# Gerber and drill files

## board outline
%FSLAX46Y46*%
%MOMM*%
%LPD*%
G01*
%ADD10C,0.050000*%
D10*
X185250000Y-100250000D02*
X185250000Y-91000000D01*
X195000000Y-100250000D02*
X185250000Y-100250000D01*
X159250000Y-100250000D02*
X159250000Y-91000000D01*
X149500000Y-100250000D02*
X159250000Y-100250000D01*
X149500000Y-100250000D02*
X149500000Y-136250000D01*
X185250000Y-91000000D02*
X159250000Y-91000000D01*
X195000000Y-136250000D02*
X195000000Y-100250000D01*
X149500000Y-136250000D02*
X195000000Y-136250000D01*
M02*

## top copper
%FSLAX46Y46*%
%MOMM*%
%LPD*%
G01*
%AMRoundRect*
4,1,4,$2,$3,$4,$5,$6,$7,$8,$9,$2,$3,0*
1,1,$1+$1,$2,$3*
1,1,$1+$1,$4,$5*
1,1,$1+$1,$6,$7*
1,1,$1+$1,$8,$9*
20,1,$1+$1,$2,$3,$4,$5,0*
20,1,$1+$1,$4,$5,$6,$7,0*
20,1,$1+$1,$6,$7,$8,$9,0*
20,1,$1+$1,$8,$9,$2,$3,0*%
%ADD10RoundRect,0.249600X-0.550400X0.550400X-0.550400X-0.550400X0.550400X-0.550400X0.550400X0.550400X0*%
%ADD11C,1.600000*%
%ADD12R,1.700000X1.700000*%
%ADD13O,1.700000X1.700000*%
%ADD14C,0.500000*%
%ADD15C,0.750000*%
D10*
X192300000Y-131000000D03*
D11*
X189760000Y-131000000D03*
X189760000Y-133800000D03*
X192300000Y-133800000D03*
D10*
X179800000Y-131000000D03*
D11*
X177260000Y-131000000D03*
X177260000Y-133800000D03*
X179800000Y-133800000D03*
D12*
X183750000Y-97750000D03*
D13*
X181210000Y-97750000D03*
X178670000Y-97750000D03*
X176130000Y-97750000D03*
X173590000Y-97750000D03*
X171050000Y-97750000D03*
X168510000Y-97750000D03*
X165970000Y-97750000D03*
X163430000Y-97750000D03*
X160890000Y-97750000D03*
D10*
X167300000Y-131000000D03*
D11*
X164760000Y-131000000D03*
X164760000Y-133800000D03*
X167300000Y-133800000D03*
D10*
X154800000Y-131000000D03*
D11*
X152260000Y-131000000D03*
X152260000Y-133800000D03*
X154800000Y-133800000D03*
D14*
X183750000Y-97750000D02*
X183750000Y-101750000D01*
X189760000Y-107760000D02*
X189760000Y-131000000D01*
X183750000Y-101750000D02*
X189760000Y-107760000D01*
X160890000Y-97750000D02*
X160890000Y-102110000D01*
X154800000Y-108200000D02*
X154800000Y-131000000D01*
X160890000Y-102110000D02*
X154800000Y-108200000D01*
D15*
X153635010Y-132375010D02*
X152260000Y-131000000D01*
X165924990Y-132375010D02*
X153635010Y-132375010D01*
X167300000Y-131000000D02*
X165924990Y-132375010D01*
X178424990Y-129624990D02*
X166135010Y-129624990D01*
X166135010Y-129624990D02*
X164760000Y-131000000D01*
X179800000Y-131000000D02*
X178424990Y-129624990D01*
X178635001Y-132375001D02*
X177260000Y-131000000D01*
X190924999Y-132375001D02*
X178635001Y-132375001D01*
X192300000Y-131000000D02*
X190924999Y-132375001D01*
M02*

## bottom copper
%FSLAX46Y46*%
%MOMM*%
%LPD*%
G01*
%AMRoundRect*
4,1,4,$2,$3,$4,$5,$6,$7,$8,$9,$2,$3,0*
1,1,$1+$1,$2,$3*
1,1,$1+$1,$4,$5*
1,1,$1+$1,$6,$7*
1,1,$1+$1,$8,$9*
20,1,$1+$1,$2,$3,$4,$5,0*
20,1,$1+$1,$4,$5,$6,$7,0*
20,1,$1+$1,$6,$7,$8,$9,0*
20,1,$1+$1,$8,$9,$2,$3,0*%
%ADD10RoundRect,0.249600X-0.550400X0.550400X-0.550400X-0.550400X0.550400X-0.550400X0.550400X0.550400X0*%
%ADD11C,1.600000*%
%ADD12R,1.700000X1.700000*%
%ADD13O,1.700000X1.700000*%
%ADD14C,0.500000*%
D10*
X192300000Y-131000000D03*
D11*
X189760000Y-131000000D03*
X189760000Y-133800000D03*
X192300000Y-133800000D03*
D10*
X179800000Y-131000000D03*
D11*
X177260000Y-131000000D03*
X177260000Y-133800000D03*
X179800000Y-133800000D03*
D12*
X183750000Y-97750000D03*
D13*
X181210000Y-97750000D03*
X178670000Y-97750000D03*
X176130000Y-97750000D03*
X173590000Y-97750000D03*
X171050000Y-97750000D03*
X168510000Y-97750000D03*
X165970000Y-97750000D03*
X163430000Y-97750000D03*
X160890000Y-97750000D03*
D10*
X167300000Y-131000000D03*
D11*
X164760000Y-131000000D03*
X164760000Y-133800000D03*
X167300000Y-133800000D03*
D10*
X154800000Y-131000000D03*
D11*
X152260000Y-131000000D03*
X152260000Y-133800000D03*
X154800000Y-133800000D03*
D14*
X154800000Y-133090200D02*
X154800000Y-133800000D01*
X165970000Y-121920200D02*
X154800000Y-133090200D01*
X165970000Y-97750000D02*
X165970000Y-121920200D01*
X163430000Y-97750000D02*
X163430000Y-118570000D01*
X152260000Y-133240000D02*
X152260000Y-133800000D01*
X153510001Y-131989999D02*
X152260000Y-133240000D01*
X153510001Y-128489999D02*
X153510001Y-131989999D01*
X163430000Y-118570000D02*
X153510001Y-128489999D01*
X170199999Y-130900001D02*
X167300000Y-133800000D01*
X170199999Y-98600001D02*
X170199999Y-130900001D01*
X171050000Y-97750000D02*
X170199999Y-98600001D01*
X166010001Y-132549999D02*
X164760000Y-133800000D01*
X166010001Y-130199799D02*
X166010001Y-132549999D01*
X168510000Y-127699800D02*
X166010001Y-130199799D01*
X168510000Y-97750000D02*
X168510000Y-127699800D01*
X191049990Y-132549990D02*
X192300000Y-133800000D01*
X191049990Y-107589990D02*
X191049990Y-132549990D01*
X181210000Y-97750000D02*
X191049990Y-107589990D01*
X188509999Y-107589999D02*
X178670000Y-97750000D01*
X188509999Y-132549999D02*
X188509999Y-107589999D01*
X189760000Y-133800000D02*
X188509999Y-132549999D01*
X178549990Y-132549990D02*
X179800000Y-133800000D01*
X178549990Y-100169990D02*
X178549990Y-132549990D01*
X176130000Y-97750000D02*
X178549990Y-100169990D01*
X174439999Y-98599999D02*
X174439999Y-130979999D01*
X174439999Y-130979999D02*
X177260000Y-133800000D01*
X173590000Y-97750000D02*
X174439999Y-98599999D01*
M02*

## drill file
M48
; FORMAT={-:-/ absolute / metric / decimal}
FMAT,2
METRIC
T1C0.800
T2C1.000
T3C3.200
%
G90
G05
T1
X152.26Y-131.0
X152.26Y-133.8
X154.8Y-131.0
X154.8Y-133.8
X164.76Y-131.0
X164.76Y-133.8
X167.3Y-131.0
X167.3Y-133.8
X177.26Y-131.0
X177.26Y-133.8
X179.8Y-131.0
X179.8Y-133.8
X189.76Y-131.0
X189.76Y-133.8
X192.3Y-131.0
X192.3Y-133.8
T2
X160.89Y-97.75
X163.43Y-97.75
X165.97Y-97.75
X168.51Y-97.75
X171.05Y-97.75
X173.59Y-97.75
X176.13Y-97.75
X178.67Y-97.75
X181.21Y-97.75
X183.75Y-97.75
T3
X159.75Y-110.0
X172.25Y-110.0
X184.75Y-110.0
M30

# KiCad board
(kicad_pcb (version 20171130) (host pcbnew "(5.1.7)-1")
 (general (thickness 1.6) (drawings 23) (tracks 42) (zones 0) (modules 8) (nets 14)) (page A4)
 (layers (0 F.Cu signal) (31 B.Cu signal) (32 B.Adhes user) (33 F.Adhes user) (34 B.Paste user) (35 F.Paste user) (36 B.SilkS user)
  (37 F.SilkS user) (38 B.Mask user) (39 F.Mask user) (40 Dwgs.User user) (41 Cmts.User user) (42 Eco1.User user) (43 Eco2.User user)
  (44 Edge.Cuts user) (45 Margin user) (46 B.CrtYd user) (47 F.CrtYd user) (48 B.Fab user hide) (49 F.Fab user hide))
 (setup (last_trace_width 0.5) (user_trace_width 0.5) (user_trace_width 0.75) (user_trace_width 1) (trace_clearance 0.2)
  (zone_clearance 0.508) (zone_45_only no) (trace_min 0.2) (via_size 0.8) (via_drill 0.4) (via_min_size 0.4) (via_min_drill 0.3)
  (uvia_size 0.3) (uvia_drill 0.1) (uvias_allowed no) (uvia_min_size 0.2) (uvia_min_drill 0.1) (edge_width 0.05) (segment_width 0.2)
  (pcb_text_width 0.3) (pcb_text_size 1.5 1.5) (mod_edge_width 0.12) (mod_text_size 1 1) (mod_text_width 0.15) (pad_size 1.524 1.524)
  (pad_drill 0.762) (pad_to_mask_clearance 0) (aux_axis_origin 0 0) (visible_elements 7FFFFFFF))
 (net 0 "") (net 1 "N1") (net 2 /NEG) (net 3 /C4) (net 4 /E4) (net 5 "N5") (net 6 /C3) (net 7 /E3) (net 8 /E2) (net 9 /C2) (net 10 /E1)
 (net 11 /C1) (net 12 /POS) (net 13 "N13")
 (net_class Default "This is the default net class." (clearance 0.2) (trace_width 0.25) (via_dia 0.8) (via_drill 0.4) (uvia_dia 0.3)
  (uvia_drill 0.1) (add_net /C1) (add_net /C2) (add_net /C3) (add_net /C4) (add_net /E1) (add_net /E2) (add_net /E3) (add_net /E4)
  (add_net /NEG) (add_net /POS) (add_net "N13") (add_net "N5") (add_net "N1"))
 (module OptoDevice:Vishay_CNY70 (layer F.Cu) (at 192.3 131 270)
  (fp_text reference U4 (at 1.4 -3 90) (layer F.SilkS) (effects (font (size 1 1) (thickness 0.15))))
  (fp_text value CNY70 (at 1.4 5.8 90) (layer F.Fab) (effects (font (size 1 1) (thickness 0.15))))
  (pad 1 thru_hole roundrect (at 0 0 270) (size 1.6 1.6) (drill 0.8) (layers *.Cu *.Mask) (roundrect_rratio 0.156) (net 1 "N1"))
  (pad 2 thru_hole circle (at 0 2.54 270) (size 1.6 1.6) (drill 0.8) (layers *.Cu *.Mask) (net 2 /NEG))
  (pad 3 thru_hole circle (at 2.8 2.54 270) (size 1.6 1.6) (drill 0.8) (layers *.Cu *.Mask) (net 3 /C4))
  (pad 4 thru_hole circle (at 2.8 0 270) (size 1.6 1.6) (drill 0.8) (layers *.Cu *.Mask) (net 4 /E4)))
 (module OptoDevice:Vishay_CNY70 (layer F.Cu) (at 179.8 131 270)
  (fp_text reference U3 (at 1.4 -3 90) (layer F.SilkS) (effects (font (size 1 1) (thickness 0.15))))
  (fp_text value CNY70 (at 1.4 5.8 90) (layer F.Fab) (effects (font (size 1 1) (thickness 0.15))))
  (pad 1 thru_hole roundrect (at 0 0 270) (size 1.6 1.6) (drill 0.8) (layers *.Cu *.Mask) (roundrect_rratio 0.156) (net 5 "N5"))
  (pad 2 thru_hole circle (at 0 2.54 270) (size 1.6 1.6) (drill 0.8) (layers *.Cu *.Mask) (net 1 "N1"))
  (pad 3 thru_hole circle (at 2.8 2.54 270) (size 1.6 1.6) (drill 0.8) (layers *.Cu *.Mask) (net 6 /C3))
  (pad 4 thru_hole circle (at 2.8 0 270) (size 1.6 1.6) (drill 0.8) (layers *.Cu *.Mask) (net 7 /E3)))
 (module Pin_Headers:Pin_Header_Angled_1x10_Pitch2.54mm (layer B.Cu) (at 183.75 97.75 90)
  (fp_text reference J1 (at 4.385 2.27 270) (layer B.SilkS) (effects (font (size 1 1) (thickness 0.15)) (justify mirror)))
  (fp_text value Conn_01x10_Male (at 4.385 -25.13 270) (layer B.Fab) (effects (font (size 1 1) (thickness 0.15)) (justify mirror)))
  (pad 1 thru_hole rect (at 0 0 90) (size 1.7 1.7) (drill 1) (layers *.Cu *.Mask) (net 2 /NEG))
  (pad 2 thru_hole oval (at 0 -2.54 90) (size 1.7 1.7) (drill 1) (layers *.Cu *.Mask) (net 4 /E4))
  (pad 3 thru_hole oval (at 0 -5.08 90) (size 1.7 1.7) (drill 1) (layers *.Cu *.Mask) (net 3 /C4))
  (pad 4 thru_hole oval (at 0 -7.62 90) (size 1.7 1.7) (drill 1) (layers *.Cu *.Mask) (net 7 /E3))
  (pad 5 thru_hole oval (at 0 -10.16 90) (size 1.7 1.7) (drill 1) (layers *.Cu *.Mask) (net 6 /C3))
  (pad 6 thru_hole oval (at 0 -12.7 90) (size 1.7 1.7) (drill 1) (layers *.Cu *.Mask) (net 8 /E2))
  (pad 7 thru_hole oval (at 0 -15.24 90) (size 1.7 1.7) (drill 1) (layers *.Cu *.Mask) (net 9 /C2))
  (pad 8 thru_hole oval (at 0 -17.78 90) (size 1.7 1.7) (drill 1) (layers *.Cu *.Mask) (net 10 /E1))
  (pad 9 thru_hole oval (at 0 -20.32 90) (size 1.7 1.7) (drill 1) (layers *.Cu *.Mask) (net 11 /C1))
  (pad 10 thru_hole oval (at 0 -22.86 90) (size 1.7 1.7) (drill 1) (layers *.Cu *.Mask) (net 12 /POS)))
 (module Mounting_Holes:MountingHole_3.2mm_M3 (layer F.Cu) (at 184.75 110)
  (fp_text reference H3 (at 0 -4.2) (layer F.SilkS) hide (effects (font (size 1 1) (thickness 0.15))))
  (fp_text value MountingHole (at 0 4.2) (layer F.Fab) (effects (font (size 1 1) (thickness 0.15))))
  (pad 1 np_thru_hole circle (at 0 0) (size 3.2 3.2) (drill 3.2) (layers *.Cu *.Mask)))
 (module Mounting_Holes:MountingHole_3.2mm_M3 (layer F.Cu) (at 172.25 110)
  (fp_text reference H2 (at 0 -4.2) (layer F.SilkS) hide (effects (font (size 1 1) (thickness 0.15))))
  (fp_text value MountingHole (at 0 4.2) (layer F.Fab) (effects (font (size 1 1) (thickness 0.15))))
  (pad 1 np_thru_hole circle (at 0 0) (size 3.2 3.2) (drill 3.2) (layers *.Cu *.Mask)))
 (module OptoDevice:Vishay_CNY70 (layer F.Cu) (at 167.3 131 270)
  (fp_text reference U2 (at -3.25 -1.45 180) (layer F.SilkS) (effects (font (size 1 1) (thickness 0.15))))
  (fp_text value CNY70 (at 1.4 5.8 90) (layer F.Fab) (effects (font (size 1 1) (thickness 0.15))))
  (pad 1 thru_hole roundrect (at 0 0 270) (size 1.6 1.6) (drill 0.8) (layers *.Cu *.Mask) (roundrect_rratio 0.156) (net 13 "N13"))
  (pad 2 thru_hole circle (at 0 2.54 270) (size 1.6 1.6) (drill 0.8) (layers *.Cu *.Mask) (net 5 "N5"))
  (pad 3 thru_hole circle (at 2.8 2.54 270) (size 1.6 1.6) (drill 0.8) (layers *.Cu *.Mask) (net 9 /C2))
  (pad 4 thru_hole circle (at 2.8 0 270) (size 1.6 1.6) (drill 0.8) (layers *.Cu *.Mask) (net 8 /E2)))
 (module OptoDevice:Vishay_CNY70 (layer F.Cu) (at 154.8 131 270)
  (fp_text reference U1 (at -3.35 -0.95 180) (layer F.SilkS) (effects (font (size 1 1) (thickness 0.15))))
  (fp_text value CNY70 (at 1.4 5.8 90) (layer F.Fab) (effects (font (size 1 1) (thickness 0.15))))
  (pad 1 thru_hole roundrect (at 0 0 270) (size 1.6 1.6) (drill 0.8) (layers *.Cu *.Mask) (roundrect_rratio 0.156) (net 12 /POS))
  (pad 2 thru_hole circle (at 0 2.54 270) (size 1.6 1.6) (drill 0.8) (layers *.Cu *.Mask) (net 13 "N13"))
  (pad 3 thru_hole circle (at 2.8 2.54 270) (size 1.6 1.6) (drill 0.8) (layers *.Cu *.Mask) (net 11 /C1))
  (pad 4 thru_hole circle (at 2.8 0 270) (size 1.6 1.6) (drill 0.8) (layers *.Cu *.Mask) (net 10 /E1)))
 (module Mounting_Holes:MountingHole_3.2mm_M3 (layer F.Cu) (at 159.75 110)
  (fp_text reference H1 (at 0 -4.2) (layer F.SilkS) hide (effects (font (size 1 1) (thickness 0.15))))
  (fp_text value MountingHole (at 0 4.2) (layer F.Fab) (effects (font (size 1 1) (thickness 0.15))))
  (pad 1 np_thru_hole circle (at 0 0) (size 3.2 3.2) (drill 3.2) (layers *.Cu *.Mask)))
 (gr_line (start 185.25 100.25) (end 185.25 91) (layer Edge.Cuts) (width 0.05))
 (gr_line (start 195 100.25) (end 185.25 100.25) (layer Edge.Cuts) (width 0.05))
 (gr_line (start 159.25 100.25) (end 159.25 91) (layer Edge.Cuts) (width 0.05))
 (gr_line (start 149.5 100.25) (end 159.25 100.25) (layer Edge.Cuts) (width 0.05))
 (gr_line (start 149.5 100.25) (end 149.5 136.25) (layer Edge.Cuts) (width 0.05))
 (gr_line (start 185.25 91) (end 159.25 91) (layer Edge.Cuts) (width 0.05))
 (gr_line (start 195 136.25) (end 195 100.25) (layer Edge.Cuts) (width 0.05))
 (gr_line (start 149.5 136.25) (end 195 136.25) (layer Edge.Cuts) (width 0.05))
 (segment (start 183.75 97.75) (end 183.75 101.75) (width 0.5) (layer F.Cu) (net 2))
 (segment (start 189.76 107.76) (end 189.76 131) (width 0.5) (layer F.Cu) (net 2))
 (segment (start 183.75 101.75) (end 189.76 107.76) (width 0.5) (layer F.Cu) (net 2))
 (segment (start 154.8 133.0902) (end 154.8 133.8) (width 0.5) (layer B.Cu) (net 10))
 (segment (start 165.97 121.9202) (end 154.8 133.0902) (width 0.5) (layer B.Cu) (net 10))
 (segment (start 165.97 97.75) (end 165.97 121.9202) (width 0.5) (layer B.Cu) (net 10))
 (segment (start 163.43 97.75) (end 163.43 118.57) (width 0.5) (layer B.Cu) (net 11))
 (segment (start 152.26 133.24) (end 152.26 133.8) (width 0.5) (layer B.Cu) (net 11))
 (segment (start 153.510001 131.989999) (end 152.26 133.24) (width 0.5) (layer B.Cu) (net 11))
 (segment (start 153.510001 128.489999) (end 153.510001 131.989999) (width 0.5) (layer B.Cu) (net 11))
 (segment (start 163.43 118.57) (end 153.510001 128.489999) (width 0.5) (layer B.Cu) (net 11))
 (segment (start 160.89 97.75) (end 160.89 102.11) (width 0.5) (layer F.Cu) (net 12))
 (segment (start 154.8 108.2) (end 154.8 131) (width 0.5) (layer F.Cu) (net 12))
 (segment (start 160.89 102.11) (end 154.8 108.2) (width 0.5) (layer F.Cu) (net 12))
 (segment (start 153.63501 132.37501) (end 152.26 131) (width 0.75) (layer F.Cu) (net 13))
 (segment (start 165.92499 132.37501) (end 153.63501 132.37501) (width 0.75) (layer F.Cu) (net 13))
 (segment (start 167.3 131) (end 165.92499 132.37501) (width 0.75) (layer F.Cu) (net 13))
 (segment (start 170.199999 130.900001) (end 167.3 133.8) (width 0.5) (layer B.Cu) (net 8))
 (segment (start 170.199999 98.600001) (end 170.199999 130.900001) (width 0.5) (layer B.Cu) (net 8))
 (segment (start 171.05 97.75) (end 170.199999 98.600001) (width 0.5) (layer B.Cu) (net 8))
 (segment (start 166.010001 132.549999) (end 164.76 133.8) (width 0.5) (layer B.Cu) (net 9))
 (segment (start 166.010001 130.199799) (end 166.010001 132.549999) (width 0.5) (layer B.Cu) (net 9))
 (segment (start 168.51 127.6998) (end 166.010001 130.199799) (width 0.5) (layer B.Cu) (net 9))
 (segment (start 168.51 97.75) (end 168.51 127.6998) (width 0.5) (layer B.Cu) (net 9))
 (segment (start 191.04999 132.54999) (end 192.3 133.8) (width 0.5) (layer B.Cu) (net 4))
 (segment (start 191.04999 107.58999) (end 191.04999 132.54999) (width 0.5) (layer B.Cu) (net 4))
 (segment (start 181.21 97.75) (end 191.04999 107.58999) (width 0.5) (layer B.Cu) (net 4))
 (segment (start 188.509999 107.589999) (end 178.67 97.75) (width 0.5) (layer B.Cu) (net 3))
 (segment (start 188.509999 132.549999) (end 188.509999 107.589999) (width 0.5) (layer B.Cu) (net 3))
 (segment (start 189.76 133.8) (end 188.509999 132.549999) (width 0.5) (layer B.Cu) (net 3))
 (segment (start 178.54999 132.54999) (end 179.8 133.8) (width 0.5) (layer B.Cu) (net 7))
 (segment (start 178.54999 100.16999) (end 178.54999 132.54999) (width 0.5) (layer B.Cu) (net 7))
 (segment (start 176.13 97.75) (end 178.54999 100.16999) (width 0.5) (layer B.Cu) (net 7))
 (segment (start 174.439999 98.599999) (end 174.439999 130.979999) (width 0.5) (layer B.Cu) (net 6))
 (segment (start 174.439999 130.979999) (end 177.26 133.8) (width 0.5) (layer B.Cu) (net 6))
 (segment (start 173.59 97.75) (end 174.439999 98.599999) (width 0.5) (layer B.Cu) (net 6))
 (segment (start 178.42499 129.62499) (end 166.13501 129.62499) (width 0.75) (layer F.Cu) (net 5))
 (segment (start 166.13501 129.62499) (end 164.76 131) (width 0.75) (layer F.Cu) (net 5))
 (segment (start 179.8 131) (end 178.42499 129.62499) (width 0.75) (layer F.Cu) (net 5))
 (segment (start 178.635001 132.375001) (end 177.26 131) (width 0.75) (layer F.Cu) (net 1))
 (segment (start 190.924999 132.375001) (end 178.635001 132.375001) (width 0.75) (layer F.Cu) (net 1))
 (segment (start 192.3 131) (end 190.924999 132.375001) (width 0.75) (layer F.Cu) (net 1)))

